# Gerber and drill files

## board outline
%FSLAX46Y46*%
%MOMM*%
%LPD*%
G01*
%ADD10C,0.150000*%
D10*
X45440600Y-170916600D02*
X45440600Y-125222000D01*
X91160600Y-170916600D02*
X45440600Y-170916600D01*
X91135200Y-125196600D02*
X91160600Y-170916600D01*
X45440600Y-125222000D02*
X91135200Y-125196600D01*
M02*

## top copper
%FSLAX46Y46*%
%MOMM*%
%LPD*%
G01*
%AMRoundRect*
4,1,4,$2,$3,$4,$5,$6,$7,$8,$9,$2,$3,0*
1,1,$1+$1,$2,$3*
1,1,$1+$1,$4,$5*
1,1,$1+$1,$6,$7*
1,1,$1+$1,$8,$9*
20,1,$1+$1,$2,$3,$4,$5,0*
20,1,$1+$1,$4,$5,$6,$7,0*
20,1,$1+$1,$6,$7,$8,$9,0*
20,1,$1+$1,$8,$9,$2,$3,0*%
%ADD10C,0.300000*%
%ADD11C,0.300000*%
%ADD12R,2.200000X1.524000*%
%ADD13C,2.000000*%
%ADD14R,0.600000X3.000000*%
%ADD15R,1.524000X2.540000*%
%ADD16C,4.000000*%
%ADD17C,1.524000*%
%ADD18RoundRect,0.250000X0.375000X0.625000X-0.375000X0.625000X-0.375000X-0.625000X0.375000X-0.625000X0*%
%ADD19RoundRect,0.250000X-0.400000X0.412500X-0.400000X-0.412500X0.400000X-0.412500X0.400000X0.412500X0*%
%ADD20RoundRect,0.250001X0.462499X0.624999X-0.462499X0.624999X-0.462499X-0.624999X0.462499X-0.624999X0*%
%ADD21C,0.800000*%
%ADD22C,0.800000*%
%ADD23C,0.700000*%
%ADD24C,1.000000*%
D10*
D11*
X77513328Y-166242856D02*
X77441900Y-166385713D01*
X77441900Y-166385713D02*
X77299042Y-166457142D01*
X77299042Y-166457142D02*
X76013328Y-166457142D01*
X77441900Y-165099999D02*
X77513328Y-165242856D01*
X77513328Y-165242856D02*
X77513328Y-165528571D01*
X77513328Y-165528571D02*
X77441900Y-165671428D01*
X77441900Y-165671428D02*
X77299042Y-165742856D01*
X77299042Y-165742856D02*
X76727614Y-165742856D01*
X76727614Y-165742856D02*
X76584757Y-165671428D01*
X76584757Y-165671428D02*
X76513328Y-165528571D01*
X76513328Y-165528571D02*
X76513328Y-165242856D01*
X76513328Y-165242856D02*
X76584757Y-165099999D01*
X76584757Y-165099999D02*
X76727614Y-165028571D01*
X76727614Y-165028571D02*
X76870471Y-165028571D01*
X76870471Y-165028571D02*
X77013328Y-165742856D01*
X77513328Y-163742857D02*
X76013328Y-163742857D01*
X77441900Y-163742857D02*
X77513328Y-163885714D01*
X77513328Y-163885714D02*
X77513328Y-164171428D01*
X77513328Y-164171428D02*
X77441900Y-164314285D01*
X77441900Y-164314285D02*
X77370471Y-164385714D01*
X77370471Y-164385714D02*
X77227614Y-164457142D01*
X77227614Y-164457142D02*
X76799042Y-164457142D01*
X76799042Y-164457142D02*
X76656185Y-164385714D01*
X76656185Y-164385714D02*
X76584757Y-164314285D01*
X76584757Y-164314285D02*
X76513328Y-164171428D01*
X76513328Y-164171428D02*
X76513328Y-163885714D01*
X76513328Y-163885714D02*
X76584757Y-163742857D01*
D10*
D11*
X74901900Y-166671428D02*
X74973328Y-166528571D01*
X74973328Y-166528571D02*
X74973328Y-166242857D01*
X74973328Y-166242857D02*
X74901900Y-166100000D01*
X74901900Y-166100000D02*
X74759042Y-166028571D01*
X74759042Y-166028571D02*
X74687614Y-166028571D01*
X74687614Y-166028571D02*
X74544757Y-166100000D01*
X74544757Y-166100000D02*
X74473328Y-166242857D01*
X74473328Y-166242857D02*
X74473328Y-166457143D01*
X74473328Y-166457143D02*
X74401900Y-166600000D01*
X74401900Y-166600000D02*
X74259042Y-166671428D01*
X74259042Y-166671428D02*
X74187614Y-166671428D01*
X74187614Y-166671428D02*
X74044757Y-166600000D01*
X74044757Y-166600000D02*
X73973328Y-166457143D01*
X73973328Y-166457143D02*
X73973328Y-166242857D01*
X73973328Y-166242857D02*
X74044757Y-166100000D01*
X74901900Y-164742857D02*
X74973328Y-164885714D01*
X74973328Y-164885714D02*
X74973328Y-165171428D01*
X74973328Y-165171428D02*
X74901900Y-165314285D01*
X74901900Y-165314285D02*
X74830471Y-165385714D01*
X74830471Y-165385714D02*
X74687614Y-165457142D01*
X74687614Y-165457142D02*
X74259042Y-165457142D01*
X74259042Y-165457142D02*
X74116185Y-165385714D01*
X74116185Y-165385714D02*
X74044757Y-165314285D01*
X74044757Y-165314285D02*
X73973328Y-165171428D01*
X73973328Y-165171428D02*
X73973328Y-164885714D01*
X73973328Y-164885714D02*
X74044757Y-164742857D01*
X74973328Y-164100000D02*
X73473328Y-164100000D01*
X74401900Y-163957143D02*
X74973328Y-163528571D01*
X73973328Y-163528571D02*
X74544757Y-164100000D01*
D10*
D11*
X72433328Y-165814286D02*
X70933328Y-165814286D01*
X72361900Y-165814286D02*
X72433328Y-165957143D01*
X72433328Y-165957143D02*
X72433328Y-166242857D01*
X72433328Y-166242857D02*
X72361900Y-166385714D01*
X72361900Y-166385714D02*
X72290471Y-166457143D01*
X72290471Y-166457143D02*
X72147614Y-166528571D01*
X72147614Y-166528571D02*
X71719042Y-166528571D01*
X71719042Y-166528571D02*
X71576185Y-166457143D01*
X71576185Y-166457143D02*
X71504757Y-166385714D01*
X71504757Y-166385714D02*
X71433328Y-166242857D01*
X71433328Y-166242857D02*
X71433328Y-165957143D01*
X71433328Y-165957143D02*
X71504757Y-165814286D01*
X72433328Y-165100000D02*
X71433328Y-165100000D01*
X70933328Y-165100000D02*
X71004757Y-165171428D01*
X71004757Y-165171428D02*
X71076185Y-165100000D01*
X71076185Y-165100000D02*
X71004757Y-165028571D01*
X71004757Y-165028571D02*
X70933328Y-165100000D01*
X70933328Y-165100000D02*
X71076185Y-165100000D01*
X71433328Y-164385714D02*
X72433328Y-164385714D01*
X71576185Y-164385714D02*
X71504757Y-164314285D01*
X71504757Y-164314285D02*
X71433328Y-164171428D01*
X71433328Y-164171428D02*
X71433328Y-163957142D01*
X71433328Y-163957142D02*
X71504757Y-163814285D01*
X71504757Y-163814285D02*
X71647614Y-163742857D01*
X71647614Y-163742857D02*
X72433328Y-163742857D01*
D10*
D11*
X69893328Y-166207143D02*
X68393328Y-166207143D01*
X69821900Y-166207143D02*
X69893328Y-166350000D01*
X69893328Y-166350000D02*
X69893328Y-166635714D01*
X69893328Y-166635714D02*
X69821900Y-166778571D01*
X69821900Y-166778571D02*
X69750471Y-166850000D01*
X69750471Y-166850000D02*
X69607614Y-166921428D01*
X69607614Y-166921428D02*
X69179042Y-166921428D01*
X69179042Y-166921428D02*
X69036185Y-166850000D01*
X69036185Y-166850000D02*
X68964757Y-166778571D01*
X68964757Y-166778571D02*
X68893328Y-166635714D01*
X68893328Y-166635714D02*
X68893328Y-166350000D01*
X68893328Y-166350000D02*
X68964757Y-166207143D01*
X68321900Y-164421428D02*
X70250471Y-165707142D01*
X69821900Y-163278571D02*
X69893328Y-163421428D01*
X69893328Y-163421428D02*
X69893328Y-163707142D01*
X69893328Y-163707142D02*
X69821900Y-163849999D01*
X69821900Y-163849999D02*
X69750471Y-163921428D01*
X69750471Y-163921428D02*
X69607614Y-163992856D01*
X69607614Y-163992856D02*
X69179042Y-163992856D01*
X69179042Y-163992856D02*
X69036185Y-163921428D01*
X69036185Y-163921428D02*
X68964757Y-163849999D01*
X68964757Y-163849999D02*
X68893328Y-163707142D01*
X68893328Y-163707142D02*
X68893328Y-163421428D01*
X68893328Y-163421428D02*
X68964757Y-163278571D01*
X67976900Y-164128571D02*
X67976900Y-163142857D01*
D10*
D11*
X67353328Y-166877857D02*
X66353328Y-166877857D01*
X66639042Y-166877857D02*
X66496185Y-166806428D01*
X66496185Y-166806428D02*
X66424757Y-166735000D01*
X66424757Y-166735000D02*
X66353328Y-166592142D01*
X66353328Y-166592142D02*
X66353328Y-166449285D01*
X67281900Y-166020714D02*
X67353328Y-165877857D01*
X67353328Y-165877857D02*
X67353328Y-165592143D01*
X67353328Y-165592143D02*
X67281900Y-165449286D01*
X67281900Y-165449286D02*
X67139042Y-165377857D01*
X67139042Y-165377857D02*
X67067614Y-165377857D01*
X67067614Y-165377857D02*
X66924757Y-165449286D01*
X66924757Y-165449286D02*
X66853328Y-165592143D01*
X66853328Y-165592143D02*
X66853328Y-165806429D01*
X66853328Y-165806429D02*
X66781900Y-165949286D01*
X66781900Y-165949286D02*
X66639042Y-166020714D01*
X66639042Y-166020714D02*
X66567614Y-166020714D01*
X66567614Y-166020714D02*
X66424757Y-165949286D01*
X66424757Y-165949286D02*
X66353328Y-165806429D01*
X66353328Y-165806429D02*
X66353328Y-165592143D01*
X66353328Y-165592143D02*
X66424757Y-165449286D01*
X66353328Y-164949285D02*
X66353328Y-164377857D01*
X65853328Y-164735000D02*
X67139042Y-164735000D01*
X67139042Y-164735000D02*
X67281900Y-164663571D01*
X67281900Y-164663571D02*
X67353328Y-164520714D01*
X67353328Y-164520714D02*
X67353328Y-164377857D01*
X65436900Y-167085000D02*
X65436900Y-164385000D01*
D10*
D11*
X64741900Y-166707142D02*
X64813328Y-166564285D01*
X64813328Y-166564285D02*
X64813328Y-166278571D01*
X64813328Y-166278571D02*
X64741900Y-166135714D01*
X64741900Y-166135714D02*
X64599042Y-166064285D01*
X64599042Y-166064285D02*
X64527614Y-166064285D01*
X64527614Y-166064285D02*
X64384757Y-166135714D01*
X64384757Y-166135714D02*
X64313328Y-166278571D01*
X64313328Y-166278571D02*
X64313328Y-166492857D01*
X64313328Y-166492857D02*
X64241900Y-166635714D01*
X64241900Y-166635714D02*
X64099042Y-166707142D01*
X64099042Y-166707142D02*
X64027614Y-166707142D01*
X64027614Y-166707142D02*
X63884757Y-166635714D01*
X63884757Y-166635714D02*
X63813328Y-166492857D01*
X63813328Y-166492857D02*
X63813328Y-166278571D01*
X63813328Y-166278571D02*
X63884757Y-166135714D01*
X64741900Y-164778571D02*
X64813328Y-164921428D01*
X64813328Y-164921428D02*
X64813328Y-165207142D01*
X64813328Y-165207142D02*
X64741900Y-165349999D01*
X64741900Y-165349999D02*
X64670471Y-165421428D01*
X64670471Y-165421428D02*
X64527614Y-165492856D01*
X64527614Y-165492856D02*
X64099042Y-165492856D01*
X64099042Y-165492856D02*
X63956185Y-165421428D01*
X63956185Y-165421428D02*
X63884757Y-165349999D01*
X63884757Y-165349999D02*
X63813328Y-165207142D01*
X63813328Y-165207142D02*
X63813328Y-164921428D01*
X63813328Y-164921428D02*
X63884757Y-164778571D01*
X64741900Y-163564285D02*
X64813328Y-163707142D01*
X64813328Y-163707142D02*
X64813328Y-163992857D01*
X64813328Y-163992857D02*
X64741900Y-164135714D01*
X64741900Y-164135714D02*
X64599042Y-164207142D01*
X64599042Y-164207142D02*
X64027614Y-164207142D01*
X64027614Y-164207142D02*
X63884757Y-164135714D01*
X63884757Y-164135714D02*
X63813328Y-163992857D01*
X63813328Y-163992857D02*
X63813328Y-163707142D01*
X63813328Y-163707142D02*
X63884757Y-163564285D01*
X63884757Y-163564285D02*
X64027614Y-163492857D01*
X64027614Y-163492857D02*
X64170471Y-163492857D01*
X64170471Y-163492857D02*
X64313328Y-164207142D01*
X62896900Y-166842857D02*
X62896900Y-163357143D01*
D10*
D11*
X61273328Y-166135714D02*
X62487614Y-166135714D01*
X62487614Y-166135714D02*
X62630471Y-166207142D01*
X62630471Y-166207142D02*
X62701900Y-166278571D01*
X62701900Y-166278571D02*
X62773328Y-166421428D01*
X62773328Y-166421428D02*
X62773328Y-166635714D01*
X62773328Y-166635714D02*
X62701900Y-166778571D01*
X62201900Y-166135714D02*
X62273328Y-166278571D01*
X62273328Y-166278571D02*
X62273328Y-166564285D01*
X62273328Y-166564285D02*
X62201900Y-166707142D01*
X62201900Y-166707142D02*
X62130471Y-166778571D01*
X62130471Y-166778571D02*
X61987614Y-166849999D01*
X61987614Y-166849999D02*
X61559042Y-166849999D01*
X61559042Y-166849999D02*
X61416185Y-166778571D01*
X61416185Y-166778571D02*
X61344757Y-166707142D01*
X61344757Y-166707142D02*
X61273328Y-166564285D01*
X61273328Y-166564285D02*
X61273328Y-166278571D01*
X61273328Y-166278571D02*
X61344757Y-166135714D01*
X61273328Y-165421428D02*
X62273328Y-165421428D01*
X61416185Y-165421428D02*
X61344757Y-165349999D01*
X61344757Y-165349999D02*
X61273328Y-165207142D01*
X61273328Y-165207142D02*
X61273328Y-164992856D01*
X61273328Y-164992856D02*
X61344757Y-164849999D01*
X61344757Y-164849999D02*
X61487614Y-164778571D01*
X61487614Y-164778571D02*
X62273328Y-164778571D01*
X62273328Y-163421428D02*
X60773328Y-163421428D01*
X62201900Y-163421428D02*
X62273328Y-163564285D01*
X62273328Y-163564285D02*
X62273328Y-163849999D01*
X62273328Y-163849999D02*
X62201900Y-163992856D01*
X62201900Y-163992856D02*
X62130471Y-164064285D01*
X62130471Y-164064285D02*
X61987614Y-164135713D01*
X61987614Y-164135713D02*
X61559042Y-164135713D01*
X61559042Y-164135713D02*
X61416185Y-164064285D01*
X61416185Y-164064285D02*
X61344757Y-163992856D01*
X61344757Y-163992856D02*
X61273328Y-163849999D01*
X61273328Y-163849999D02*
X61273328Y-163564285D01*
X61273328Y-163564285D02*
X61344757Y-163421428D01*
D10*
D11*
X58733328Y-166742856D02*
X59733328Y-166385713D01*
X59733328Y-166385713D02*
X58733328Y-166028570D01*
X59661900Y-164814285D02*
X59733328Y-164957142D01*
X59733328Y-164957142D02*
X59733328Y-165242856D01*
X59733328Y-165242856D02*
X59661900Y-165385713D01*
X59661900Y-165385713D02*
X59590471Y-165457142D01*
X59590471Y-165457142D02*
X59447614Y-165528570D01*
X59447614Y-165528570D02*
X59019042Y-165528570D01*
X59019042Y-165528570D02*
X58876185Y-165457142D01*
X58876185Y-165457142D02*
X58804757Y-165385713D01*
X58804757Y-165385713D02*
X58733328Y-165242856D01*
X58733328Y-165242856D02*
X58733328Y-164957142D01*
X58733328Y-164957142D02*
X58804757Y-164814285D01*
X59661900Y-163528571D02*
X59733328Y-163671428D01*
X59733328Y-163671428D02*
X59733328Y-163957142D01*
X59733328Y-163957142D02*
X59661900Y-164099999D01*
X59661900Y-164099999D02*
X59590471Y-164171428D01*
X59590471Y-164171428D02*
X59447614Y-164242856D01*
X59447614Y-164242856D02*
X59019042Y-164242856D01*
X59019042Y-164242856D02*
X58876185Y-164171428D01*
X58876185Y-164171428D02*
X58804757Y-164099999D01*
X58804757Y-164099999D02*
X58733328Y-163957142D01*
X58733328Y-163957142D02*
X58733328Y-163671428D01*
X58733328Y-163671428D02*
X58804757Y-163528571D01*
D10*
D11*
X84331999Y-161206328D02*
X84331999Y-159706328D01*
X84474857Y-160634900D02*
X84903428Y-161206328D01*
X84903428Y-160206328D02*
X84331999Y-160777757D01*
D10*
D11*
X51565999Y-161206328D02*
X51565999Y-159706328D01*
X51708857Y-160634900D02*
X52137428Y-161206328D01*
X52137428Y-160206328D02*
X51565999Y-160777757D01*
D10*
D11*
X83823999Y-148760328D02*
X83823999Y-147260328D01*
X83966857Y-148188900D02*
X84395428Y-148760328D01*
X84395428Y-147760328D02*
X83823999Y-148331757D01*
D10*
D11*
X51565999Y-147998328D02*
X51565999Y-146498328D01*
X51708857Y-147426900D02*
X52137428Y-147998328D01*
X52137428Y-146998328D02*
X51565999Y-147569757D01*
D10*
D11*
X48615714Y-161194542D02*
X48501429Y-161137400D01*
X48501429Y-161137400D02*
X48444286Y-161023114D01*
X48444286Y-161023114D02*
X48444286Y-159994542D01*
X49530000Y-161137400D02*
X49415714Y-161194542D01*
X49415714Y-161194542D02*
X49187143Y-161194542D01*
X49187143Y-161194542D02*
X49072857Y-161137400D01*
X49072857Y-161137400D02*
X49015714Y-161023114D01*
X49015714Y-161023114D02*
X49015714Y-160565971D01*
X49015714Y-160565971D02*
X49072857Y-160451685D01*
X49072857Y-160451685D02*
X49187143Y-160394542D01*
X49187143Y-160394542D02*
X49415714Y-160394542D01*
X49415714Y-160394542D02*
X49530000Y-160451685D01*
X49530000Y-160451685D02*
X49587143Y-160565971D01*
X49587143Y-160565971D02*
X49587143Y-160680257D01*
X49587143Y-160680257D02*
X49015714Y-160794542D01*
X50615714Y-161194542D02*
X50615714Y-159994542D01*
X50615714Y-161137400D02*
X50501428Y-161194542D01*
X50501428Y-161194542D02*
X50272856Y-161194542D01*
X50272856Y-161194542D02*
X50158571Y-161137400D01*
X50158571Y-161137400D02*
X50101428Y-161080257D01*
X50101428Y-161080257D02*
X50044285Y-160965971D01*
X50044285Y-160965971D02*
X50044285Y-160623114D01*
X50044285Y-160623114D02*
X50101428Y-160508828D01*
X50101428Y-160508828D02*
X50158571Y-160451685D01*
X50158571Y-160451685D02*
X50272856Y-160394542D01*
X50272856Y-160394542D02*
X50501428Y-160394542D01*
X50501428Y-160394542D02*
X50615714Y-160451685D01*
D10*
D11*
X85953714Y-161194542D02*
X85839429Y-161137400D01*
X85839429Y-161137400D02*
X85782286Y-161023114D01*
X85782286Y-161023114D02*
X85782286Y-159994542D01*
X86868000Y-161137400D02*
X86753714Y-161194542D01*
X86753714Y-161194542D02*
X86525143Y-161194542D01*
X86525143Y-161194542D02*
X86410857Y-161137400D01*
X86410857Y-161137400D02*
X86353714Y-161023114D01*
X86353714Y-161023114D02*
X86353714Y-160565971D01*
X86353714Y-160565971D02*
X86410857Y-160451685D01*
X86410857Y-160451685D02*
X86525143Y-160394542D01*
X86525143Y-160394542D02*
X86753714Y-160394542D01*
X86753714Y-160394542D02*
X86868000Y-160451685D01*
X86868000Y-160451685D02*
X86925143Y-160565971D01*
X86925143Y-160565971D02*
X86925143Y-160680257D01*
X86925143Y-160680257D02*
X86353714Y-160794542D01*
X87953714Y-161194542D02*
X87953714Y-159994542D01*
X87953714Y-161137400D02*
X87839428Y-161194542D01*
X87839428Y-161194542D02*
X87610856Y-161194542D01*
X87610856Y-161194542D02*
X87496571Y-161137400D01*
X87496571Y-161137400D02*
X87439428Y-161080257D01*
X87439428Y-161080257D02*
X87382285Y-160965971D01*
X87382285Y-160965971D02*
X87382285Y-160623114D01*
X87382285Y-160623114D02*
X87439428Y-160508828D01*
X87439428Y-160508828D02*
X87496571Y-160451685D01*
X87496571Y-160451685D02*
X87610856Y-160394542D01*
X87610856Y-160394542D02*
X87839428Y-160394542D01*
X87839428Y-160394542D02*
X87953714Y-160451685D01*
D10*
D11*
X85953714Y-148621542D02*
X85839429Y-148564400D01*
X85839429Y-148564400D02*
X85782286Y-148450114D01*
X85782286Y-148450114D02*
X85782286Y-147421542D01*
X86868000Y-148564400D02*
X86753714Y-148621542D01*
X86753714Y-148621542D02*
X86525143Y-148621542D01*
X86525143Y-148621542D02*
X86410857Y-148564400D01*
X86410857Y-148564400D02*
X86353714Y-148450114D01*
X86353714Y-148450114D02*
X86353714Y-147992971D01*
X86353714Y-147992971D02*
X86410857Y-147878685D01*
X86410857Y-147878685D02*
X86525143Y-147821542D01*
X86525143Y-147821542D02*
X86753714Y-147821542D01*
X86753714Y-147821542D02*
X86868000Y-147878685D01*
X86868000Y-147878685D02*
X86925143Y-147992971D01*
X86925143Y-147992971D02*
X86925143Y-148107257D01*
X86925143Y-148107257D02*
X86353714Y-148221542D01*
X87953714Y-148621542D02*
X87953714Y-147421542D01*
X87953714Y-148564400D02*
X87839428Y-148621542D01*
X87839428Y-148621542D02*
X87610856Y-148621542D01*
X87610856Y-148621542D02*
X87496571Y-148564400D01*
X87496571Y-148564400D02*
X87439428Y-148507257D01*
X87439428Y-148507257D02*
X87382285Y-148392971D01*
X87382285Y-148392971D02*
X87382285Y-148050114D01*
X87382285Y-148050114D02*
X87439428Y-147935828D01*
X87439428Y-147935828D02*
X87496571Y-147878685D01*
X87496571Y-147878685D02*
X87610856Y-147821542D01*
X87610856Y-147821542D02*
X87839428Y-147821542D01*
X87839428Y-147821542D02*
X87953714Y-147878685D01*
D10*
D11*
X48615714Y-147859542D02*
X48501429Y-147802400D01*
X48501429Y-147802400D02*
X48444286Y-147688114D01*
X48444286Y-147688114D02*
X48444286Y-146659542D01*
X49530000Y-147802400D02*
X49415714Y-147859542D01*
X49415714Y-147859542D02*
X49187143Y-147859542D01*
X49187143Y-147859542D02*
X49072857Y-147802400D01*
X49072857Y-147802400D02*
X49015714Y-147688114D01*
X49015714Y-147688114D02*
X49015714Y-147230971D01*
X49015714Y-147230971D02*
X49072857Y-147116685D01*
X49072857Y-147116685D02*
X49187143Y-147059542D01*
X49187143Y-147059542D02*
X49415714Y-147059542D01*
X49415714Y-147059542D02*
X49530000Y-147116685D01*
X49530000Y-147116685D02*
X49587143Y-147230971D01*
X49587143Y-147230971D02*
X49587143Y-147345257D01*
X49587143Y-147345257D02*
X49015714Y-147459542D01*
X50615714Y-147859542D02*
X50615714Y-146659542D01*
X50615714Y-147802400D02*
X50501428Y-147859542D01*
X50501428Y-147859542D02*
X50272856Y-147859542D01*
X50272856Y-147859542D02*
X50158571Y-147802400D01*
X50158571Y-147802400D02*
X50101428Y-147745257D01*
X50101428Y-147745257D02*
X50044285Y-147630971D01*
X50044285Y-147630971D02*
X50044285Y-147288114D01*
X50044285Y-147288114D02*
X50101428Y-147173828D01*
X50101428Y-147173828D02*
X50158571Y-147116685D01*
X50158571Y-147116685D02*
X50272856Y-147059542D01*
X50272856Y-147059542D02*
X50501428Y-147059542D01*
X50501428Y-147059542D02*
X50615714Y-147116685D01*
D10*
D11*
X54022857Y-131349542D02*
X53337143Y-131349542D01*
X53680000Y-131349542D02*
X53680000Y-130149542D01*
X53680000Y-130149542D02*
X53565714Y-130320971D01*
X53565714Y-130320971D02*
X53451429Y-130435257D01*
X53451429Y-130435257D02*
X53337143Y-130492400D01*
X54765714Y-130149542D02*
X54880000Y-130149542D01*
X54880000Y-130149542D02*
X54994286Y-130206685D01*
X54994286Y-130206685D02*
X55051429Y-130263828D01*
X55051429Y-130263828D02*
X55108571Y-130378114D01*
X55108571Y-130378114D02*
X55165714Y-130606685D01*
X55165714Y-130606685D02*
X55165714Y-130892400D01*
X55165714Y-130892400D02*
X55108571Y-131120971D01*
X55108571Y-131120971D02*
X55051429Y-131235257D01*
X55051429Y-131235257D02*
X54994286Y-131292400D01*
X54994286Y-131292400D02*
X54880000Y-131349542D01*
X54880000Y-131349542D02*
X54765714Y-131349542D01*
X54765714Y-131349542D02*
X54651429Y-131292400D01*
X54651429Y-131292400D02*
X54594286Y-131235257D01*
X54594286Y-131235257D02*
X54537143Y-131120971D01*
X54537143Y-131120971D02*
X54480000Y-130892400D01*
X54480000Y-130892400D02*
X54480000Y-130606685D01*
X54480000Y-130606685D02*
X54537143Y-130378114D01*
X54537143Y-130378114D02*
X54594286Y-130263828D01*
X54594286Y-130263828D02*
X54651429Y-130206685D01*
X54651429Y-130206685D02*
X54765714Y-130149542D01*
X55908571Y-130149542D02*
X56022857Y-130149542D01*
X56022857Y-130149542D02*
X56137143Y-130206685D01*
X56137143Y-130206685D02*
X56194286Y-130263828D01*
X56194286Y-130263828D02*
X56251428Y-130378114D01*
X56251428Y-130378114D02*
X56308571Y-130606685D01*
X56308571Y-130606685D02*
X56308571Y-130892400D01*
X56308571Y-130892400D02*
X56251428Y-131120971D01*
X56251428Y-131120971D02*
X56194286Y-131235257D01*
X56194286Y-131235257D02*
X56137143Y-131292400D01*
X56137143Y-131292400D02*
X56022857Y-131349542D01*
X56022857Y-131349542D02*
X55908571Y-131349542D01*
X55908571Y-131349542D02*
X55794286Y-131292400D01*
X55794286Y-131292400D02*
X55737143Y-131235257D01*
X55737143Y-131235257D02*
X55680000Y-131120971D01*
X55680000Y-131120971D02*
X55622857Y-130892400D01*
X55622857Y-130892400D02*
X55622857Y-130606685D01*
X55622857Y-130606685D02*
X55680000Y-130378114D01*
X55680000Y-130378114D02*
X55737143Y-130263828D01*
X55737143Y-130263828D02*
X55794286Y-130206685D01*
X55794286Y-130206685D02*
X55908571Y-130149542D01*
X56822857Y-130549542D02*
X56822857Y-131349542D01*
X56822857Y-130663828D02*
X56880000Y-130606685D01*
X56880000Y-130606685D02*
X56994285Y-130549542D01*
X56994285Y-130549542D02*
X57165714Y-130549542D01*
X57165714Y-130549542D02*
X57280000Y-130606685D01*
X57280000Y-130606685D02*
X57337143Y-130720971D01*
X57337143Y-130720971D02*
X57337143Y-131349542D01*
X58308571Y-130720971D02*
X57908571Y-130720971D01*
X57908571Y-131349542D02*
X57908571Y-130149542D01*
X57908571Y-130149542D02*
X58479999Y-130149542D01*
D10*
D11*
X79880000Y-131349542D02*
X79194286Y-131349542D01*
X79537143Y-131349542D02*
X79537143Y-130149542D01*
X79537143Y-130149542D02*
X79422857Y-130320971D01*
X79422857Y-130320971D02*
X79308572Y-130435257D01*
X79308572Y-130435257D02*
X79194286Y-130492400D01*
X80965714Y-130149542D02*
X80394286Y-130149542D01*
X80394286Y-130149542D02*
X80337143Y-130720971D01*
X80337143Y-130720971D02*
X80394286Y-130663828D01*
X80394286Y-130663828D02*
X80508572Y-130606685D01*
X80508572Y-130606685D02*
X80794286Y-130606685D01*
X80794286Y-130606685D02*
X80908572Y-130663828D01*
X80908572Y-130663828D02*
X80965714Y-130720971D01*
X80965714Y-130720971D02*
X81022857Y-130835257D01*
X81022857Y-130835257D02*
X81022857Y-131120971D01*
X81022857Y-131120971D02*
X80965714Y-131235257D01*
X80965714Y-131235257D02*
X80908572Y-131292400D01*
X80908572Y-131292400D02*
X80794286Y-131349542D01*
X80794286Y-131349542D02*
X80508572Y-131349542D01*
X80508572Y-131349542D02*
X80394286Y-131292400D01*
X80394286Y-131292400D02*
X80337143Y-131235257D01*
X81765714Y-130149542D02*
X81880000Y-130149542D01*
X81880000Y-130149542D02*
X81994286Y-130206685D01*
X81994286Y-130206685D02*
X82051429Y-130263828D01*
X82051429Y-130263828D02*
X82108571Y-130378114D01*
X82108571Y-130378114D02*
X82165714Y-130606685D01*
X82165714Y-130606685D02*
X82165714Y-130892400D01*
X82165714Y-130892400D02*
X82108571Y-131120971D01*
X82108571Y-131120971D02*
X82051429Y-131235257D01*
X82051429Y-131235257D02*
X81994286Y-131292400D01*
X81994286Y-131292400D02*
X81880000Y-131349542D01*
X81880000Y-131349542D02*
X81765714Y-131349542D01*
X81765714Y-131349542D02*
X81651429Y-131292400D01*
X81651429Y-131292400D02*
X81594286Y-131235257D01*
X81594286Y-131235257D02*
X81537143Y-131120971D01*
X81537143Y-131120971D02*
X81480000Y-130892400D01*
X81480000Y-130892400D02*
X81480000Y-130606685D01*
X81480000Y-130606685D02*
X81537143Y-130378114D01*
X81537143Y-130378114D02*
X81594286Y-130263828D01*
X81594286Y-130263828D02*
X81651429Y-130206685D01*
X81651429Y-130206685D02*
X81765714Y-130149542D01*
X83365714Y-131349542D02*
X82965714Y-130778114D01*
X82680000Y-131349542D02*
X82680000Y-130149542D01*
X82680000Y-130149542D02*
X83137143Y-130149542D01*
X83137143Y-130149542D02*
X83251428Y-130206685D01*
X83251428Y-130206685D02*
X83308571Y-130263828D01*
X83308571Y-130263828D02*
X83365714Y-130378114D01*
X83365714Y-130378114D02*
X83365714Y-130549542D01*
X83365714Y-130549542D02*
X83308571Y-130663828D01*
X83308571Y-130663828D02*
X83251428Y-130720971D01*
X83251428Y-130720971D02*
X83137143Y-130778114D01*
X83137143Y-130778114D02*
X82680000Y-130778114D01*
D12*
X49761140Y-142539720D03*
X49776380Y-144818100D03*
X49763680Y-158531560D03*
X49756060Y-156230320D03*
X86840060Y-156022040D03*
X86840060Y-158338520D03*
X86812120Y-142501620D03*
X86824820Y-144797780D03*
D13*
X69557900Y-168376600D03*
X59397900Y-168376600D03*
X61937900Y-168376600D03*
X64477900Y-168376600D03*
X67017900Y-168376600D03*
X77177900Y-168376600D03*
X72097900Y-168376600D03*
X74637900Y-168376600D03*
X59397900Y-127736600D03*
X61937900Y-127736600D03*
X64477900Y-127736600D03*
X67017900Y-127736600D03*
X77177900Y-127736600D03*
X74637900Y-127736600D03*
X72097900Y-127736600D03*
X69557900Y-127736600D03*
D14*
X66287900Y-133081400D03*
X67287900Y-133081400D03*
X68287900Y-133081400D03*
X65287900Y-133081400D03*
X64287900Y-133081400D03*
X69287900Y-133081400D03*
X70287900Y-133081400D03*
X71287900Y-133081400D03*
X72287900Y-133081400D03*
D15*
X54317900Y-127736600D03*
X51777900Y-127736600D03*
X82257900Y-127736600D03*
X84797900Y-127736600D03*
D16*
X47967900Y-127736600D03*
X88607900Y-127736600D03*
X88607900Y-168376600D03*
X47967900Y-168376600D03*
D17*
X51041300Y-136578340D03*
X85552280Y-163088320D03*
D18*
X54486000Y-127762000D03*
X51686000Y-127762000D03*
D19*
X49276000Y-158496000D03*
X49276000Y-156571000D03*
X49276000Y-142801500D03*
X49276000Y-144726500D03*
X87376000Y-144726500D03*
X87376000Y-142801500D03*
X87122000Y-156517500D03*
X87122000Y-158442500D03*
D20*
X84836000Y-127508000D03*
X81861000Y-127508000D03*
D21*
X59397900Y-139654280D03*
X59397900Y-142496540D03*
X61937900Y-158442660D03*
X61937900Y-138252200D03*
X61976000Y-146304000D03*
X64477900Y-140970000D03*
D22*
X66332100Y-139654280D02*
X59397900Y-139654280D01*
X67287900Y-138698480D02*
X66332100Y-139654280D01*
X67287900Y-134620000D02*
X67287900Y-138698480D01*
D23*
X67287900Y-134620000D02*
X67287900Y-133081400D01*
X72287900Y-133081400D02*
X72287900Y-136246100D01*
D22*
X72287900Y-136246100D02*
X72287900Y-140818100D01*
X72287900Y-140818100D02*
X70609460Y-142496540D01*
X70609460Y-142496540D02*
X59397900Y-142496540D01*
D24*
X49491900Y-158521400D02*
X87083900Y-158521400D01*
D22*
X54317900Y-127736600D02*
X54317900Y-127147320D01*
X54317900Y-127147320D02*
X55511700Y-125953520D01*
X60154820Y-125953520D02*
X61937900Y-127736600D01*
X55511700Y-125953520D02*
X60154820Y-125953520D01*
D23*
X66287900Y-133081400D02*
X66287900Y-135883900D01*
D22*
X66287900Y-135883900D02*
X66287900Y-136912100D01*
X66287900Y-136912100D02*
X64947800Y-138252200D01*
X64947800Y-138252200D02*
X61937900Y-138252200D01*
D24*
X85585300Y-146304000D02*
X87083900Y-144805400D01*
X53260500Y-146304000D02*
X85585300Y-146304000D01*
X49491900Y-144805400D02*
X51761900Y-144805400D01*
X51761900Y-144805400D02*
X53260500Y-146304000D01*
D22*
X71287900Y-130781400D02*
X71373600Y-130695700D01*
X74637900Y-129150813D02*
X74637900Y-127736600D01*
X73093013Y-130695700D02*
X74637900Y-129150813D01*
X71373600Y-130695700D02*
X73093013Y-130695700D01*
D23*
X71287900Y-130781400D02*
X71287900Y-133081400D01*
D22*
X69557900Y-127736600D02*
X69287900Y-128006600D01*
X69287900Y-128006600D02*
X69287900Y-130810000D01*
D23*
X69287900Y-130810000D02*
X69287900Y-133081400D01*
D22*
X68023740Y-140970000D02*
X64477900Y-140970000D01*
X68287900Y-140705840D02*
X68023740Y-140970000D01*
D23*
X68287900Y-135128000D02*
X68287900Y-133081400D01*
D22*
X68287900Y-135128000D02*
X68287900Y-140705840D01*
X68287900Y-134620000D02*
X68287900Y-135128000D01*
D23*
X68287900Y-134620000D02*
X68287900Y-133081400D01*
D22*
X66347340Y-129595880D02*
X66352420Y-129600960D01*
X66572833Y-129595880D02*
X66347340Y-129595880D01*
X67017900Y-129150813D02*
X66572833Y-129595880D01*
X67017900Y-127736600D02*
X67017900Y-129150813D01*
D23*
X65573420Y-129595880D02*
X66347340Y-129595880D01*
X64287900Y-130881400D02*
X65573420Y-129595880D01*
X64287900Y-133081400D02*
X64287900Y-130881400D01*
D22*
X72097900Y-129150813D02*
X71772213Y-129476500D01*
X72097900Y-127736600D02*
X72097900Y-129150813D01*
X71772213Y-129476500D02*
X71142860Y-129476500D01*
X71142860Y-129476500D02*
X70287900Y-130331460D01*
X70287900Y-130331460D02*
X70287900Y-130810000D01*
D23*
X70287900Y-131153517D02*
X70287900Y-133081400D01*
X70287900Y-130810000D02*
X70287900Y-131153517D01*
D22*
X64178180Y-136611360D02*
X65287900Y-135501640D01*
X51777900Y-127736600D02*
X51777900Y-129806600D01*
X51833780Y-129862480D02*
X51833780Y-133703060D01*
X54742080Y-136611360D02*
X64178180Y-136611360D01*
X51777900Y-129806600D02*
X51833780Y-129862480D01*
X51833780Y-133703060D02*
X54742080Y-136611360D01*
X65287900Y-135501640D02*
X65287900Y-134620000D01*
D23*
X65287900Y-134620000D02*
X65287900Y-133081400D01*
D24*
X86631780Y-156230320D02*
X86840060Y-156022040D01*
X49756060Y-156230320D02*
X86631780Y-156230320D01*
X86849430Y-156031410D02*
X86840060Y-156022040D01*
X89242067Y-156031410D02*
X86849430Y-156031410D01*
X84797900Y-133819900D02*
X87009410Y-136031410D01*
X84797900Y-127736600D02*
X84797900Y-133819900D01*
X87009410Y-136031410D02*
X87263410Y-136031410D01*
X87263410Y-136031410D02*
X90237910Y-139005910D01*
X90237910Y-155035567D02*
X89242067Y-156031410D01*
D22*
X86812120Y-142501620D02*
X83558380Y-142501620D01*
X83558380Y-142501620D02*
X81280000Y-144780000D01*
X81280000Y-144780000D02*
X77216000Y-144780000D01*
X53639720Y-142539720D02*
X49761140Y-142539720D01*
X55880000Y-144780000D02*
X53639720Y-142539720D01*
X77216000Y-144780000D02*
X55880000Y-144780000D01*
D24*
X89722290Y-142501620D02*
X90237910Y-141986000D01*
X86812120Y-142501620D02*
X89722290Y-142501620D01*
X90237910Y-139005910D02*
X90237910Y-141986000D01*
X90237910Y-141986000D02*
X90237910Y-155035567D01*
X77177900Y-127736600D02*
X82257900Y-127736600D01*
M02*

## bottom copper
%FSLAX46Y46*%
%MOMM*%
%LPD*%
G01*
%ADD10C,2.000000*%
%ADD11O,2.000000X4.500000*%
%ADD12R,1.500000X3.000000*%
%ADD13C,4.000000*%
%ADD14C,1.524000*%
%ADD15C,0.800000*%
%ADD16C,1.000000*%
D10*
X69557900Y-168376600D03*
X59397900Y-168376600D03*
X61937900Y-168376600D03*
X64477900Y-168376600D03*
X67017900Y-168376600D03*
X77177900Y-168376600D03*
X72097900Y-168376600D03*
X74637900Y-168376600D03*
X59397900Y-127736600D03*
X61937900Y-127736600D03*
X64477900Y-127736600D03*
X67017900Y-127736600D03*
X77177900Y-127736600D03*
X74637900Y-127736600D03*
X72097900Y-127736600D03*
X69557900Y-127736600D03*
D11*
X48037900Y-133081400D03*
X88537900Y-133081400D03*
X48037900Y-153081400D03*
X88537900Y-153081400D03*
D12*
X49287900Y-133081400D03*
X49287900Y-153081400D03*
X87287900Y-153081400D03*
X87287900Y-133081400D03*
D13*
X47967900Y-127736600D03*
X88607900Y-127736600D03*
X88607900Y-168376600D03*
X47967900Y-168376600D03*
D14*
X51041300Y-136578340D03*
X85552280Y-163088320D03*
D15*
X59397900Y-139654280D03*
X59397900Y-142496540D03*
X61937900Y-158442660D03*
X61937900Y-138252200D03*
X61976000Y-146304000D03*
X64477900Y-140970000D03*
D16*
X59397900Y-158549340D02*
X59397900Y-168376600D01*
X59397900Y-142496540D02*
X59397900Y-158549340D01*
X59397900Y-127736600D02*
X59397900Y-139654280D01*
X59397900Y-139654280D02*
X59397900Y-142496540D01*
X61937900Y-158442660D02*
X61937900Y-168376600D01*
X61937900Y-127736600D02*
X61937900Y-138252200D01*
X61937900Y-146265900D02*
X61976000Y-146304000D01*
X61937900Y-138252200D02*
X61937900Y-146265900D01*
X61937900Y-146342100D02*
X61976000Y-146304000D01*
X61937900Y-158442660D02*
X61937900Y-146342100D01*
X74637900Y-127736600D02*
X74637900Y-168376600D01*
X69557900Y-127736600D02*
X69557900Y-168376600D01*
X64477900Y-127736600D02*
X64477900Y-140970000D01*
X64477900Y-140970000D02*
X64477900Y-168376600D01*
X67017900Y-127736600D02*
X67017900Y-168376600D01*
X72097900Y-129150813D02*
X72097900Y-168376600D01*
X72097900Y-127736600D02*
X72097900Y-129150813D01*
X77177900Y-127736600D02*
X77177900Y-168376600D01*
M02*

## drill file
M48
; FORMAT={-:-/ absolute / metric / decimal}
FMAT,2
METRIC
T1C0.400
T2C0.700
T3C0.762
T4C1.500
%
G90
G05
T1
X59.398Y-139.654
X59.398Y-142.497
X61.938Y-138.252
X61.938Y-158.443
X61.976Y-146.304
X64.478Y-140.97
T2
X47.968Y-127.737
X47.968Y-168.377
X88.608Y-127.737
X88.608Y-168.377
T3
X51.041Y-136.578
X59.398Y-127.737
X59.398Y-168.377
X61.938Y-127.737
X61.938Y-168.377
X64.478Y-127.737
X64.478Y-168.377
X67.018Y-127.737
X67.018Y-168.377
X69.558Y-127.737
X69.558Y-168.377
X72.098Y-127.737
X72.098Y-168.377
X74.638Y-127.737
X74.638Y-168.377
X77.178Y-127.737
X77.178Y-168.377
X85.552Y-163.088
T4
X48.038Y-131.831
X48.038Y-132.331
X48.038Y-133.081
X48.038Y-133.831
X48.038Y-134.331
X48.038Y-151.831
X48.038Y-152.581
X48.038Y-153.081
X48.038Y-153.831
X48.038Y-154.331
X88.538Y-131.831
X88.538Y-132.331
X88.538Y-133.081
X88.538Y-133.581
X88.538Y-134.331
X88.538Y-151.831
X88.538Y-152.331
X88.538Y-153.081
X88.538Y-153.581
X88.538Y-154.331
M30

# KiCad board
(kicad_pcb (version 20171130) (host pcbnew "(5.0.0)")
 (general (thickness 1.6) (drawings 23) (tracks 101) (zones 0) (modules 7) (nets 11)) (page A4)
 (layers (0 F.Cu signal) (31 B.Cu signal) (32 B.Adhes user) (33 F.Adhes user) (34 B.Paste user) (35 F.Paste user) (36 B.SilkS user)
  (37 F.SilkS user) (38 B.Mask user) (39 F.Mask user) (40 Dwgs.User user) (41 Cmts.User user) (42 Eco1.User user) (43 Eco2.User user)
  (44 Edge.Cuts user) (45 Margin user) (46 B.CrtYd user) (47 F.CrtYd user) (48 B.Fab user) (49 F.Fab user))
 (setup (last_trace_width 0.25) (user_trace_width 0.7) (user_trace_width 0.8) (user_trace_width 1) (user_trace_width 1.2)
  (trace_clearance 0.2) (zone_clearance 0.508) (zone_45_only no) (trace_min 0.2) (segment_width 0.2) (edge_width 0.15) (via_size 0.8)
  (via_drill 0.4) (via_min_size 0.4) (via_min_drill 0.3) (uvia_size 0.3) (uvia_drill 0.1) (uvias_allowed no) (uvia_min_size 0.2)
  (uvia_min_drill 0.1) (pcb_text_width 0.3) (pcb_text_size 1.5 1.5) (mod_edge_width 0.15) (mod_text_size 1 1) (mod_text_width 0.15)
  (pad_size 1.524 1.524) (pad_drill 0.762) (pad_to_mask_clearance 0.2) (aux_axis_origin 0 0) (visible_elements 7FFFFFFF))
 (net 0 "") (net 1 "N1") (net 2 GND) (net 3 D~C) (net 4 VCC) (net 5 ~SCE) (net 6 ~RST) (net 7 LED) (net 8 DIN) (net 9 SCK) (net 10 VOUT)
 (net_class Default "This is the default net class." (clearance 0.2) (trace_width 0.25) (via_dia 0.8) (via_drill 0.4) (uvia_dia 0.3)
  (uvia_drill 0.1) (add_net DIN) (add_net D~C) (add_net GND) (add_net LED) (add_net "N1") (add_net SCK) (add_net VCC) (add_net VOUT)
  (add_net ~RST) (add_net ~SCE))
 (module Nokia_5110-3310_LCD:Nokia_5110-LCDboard (layer F.Cu) (at 68.2879 146.7866)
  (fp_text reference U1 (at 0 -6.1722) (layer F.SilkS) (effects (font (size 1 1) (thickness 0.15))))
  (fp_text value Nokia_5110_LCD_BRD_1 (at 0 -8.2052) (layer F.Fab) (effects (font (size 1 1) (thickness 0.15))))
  (pad 15 smd rect (at -18.52676 -4.24688 180) (size 2.2 1.524) (layers F.Cu F.Paste F.Mask) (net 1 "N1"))
  (pad 16 smd rect (at -18.51152 -1.9685) (size 2.2 1.524) (layers F.Cu F.Paste F.Mask) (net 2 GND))
  (pad 18 smd rect (at -18.52422 11.74496) (size 2.2 1.524) (layers F.Cu F.Paste F.Mask) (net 2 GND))
  (pad 17 smd rect (at -18.53184 9.44372) (size 2.2 1.524) (layers F.Cu F.Paste F.Mask) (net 1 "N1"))
  (pad 21 smd rect (at 18.55216 9.23544) (size 2.2 1.524) (layers F.Cu F.Paste F.Mask) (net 1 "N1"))
  (pad 22 smd rect (at 18.55216 11.55192) (size 2.2 1.524) (layers F.Cu F.Paste F.Mask) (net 2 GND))
  (pad 19 smd rect (at 18.52422 -4.28498) (size 2.2 1.524) (layers F.Cu F.Paste F.Mask) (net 1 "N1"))
  (pad 20 smd rect (at 18.53692 -1.98882) (size 2.2 1.524) (layers F.Cu F.Paste F.Mask) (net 2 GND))
  (pad 45 thru_hole circle (at 1.27 21.59) (size 2 2) (drill 0.762) (layers *.Cu *.Mask) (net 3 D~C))
  (pad 41 thru_hole circle (at -8.89 21.59) (size 2 2) (drill 0.762) (layers *.Cu *.Mask) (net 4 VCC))
  (pad 42 thru_hole circle (at -6.35 21.59) (size 2 2) (drill 0.762) (layers *.Cu *.Mask) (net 2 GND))
  (pad 43 thru_hole circle (at -3.81 21.59) (size 2 2) (drill 0.762) (layers *.Cu *.Mask) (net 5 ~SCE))
  (pad 44 thru_hole circle (at -1.27 21.59) (size 2 2) (drill 0.762) (layers *.Cu *.Mask) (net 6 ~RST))
  (pad 48 thru_hole circle (at 8.89 21.59) (size 2 2) (drill 0.762) (layers *.Cu *.Mask) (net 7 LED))
  (pad 46 thru_hole circle (at 3.81 21.59) (size 2 2) (drill 0.762) (layers *.Cu *.Mask) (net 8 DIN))
  (pad 47 thru_hole circle (at 6.35 21.59) (size 2 2) (drill 0.762) (layers *.Cu *.Mask) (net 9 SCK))
  (pad 31 thru_hole circle (at -8.89 -19.05) (size 2 2) (drill 0.762) (layers *.Cu *.Mask) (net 4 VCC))
  (pad 32 thru_hole circle (at -6.35 -19.05) (size 2 2) (drill 0.762) (layers *.Cu *.Mask) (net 2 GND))
  (pad 33 thru_hole circle (at -3.81 -19.05) (size 2 2) (drill 0.762) (layers *.Cu *.Mask) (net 5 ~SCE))
  (pad 34 thru_hole circle (at -1.27 -19.05) (size 2 2) (drill 0.762) (layers *.Cu *.Mask) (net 6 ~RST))
  (pad 38 thru_hole circle (at 8.89 -19.05) (size 2 2) (drill 0.762) (layers *.Cu *.Mask) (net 7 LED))
  (pad 37 thru_hole circle (at 6.35 -19.05) (size 2 2) (drill 0.762) (layers *.Cu *.Mask) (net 9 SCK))
  (pad 36 thru_hole circle (at 3.81 -19.05) (size 2 2) (drill 0.762) (layers *.Cu *.Mask) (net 8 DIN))
  (pad 35 thru_hole circle (at 1.27 -19.05) (size 2 2) (drill 0.762) (layers *.Cu *.Mask) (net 3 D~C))
  (pad "" np_thru_hole circle (at 20.25 -14.4552) (size 1.5 1.5) (drill 1.5) (layers *.Mask B.Cu F.SilkS))
  (pad "" np_thru_hole circle (at 20.25 -12.4552) (size 1.5 1.5) (drill 1.5) (layers *.Mask B.Cu F.SilkS))
  (pad "" np_thru_hole circle (at 20.25 -14.9552) (size 1.5 1.5) (drill 1.5) (layers *.Mask B.Cu F.SilkS))
  (pad 3 smd rect (at -2 -13.7052) (size 0.6 3) (layers F.Cu F.Paste F.Mask) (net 2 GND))
  (pad 4 smd rect (at -1 -13.7052) (size 0.6 3) (layers F.Cu F.Paste F.Mask) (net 4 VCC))
  (pad 5 smd rect (at 0 -13.7052) (size 0.6 3) (layers F.Cu F.Paste F.Mask) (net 5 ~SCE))
  (pad 2 smd rect (at -3 -13.7052) (size 0.6 3) (layers F.Cu F.Paste F.Mask) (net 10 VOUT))
  (pad 1 smd rect (at -4 -13.7052) (size 0.6 3) (layers F.Cu F.Paste F.Mask) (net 6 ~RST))
  (pad 6 smd rect (at 1 -13.7052) (size 0.6 3) (layers F.Cu F.Paste F.Mask) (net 3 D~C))
  (pad 7 smd rect (at 2 -13.7052) (size 0.6 3) (layers F.Cu F.Paste F.Mask) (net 8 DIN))
  (pad 8 smd rect (at 3 -13.7052) (size 0.6 3) (layers F.Cu F.Paste F.Mask) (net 9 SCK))
  (pad 9 smd rect (at 4 -13.7052) (size 0.6 3) (layers F.Cu F.Paste F.Mask) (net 4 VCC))
  (pad "" np_thru_hole oval (at -20.25 -13.7052) (size 2 4.5) (drill 1.5) (layers *.Mask B.Cu F.SilkS))
  (pad "" np_thru_hole oval (at 20.25 -13.7052) (size 2 4.5) (drill 1.5) (layers *.Mask B.Cu F.SilkS))
  (pad "" np_thru_hole oval (at -20.25 6.2948) (size 2 4.5) (drill 1.5) (layers *.Mask B.Cu F.SilkS))
  (pad "" np_thru_hole oval (at 20.25 6.2948) (size 2 4.5) (drill 1.5) (layers *.Mask B.Cu F.SilkS))
  (pad "" smd rect (at -19 -13.7052) (size 1.5 3) (layers B.Cu B.Paste B.Mask))
  (pad "" smd rect (at -19 6.2948) (size 1.5 3) (layers B.Cu B.Paste B.Mask))
  (pad "" smd rect (at 19 6.2948) (size 1.5 3) (layers B.Cu B.Paste B.Mask))
  (pad "" smd rect (at 19 -13.7052) (size 1.5 3) (layers B.Cu B.Paste B.Mask))
  (pad "" np_thru_hole circle (at 20.25 -13.2052) (size 1.5 1.5) (drill 1.5) (layers *.Mask B.Cu F.SilkS))
  (pad "" np_thru_hole circle (at 20.25 5.0448) (size 1.5 1.5) (drill 1.5) (layers *.Mask B.Cu F.SilkS))
  (pad "" np_thru_hole circle (at 20.25 7.5448) (size 1.5 1.5) (drill 1.5) (layers *.Mask B.Cu F.SilkS))
  (pad "" np_thru_hole circle (at -20.25 -14.4552) (size 1.5 1.5) (drill 1.5) (layers *.Mask B.Cu F.SilkS))
  (pad "" np_thru_hole circle (at -20.25 -14.9552) (size 1.5 1.5) (drill 1.5) (layers *.Mask B.Cu F.SilkS))
  (pad "" np_thru_hole circle (at -20.25 -12.9552) (size 1.5 1.5) (drill 1.5) (layers *.Mask B.Cu F.SilkS))
  (pad "" np_thru_hole circle (at -20.25 -12.4552) (size 1.5 1.5) (drill 1.5) (layers *.Mask B.Cu F.SilkS))
  (pad "" np_thru_hole circle (at -20.25 5.0448) (size 1.5 1.5) (drill 1.5) (layers *.Mask B.Cu F.SilkS))
  (pad "" np_thru_hole circle (at -20.25 7.5448) (size 1.5 1.5) (drill 1.5) (layers *.Mask B.Cu F.SilkS))
  (pad "" np_thru_hole circle (at -20.25 5.7948) (size 1.5 1.5) (drill 1.5) (layers *.Mask B.Cu F.SilkS))
  (pad "" np_thru_hole circle (at -20.25 7.0448) (size 1.5 1.5) (drill 1.5) (layers *.Mask B.Cu F.SilkS))
  (pad "" np_thru_hole circle (at 20.25 5.5448) (size 1.5 1.5) (drill 1.5) (layers *.Mask B.Cu F.SilkS))
  (pad "" np_thru_hole circle (at 20.25 6.7948) (size 1.5 1.5) (drill 1.5) (layers *.Mask B.Cu F.SilkS))
  (pad 12 smd rect (at -13.97 -19.05 90) (size 2.54 1.524) (layers F.Cu F.Paste F.Mask) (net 2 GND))
  (pad 11 smd rect (at -16.51 -19.05 90) (size 2.54 1.524) (layers F.Cu F.Paste F.Mask) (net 10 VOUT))
  (pad 13 smd rect (at 13.97 -19.05 90) (size 2.54 1.524) (layers F.Cu F.Paste F.Mask) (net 7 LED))
  (pad 14 smd rect (at 16.51 -19.05 90) (size 2.54 1.524) (layers F.Cu F.Paste F.Mask) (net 1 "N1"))
  (pad 01 thru_hole circle (at -20.32 -19.05 90) (size 4 4) (drill 0.7) (layers *.Cu *.Adhes *.Paste *.Mask))
  (pad 02 thru_hole circle (at 20.32 -19.05 90) (size 4 4) (drill 0.7) (layers *.Cu *.Adhes *.Paste *.Mask))
  (pad 04 thru_hole circle (at 20.32 21.59 90) (size 4 4) (drill 0.7) (layers *.Cu *.Adhes *.Paste *.Mask))
  (pad 03 thru_hole circle (at -20.32 21.59 90) (size 4 4) (drill 0.7) (layers *.Cu *.Adhes *.Paste *.Mask))
  (pad 10 thru_hole circle (at -17.2466 -10.20826) (size 1.524 1.524) (drill 0.762) (layers *.Cu *.Mask))
  (pad 23 thru_hole circle (at 17.26438 16.30172) (size 1.524 1.524) (drill 0.762) (layers *.Cu *.Mask)))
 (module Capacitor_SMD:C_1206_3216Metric (layer F.Cu) (at 53.086 127.762 180)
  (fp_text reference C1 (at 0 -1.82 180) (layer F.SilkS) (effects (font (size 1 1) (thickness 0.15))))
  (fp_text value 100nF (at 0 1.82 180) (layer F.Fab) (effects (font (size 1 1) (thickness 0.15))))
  (pad 1 smd roundrect (at -1.4 0 180) (size 1.25 1.75) (layers F.Cu F.Paste F.Mask) (roundrect_rratio 0.2) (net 2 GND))
  (pad 2 smd roundrect (at 1.4 0 180) (size 1.25 1.75) (layers F.Cu F.Paste F.Mask) (roundrect_rratio 0.2) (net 10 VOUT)))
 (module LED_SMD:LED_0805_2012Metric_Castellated (layer F.Cu) (at 49.276 157.5335 270)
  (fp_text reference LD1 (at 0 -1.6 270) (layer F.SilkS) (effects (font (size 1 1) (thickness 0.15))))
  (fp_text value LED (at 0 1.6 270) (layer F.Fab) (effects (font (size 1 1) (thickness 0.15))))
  (pad 2 smd roundrect (at 0.9625 0 270) (size 1.325 1.3) (layers F.Cu F.Paste F.Mask) (roundrect_rratio 0.192308) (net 2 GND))
  (pad 1 smd roundrect (at -0.9625 0 270) (size 1.325 1.3) (layers F.Cu F.Paste F.Mask) (roundrect_rratio 0.192308) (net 1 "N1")))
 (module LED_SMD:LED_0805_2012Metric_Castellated (layer F.Cu) (at 49.276 143.764 270)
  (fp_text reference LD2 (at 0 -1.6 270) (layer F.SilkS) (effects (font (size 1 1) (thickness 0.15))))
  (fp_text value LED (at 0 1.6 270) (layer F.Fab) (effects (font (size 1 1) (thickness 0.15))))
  (pad 1 smd roundrect (at -0.9625 0 270) (size 1.325 1.3) (layers F.Cu F.Paste F.Mask) (roundrect_rratio 0.192308) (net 1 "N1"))
  (pad 2 smd roundrect (at 0.9625 0 270) (size 1.325 1.3) (layers F.Cu F.Paste F.Mask) (roundrect_rratio 0.192308) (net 2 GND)))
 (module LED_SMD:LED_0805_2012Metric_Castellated (layer F.Cu) (at 87.376 143.764 270)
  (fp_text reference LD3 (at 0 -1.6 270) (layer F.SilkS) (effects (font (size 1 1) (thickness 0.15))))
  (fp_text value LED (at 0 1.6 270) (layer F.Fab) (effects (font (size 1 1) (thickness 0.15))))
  (pad 2 smd roundrect (at 0.9625 0 270) (size 1.325 1.3) (layers F.Cu F.Paste F.Mask) (roundrect_rratio 0.192308) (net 2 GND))
  (pad 1 smd roundrect (at -0.9625 0 270) (size 1.325 1.3) (layers F.Cu F.Paste F.Mask) (roundrect_rratio 0.192308) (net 1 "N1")))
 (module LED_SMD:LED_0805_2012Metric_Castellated (layer F.Cu) (at 87.122 157.48 270)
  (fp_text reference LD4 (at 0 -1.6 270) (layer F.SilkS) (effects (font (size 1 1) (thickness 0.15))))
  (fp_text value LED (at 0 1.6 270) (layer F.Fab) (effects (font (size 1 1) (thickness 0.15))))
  (pad 1 smd roundrect (at -0.9625 0 270) (size 1.325 1.3) (layers F.Cu F.Paste F.Mask) (roundrect_rratio 0.192308) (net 1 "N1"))
  (pad 2 smd roundrect (at 0.9625 0 270) (size 1.325 1.3) (layers F.Cu F.Paste F.Mask) (roundrect_rratio 0.192308) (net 2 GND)))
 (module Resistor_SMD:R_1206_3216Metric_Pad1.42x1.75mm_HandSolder (layer F.Cu) (at 83.3485 127.508 180)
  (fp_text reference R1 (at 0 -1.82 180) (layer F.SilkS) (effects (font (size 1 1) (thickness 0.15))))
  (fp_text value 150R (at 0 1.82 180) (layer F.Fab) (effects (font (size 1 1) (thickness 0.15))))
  (pad 1 smd roundrect (at -1.4875 0 180) (size 1.425 1.75) (layers F.Cu F.Paste F.Mask) (roundrect_rratio 0.175439) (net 1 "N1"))
  (pad 2 smd roundrect (at 1.4875 0 180) (size 1.425 1.75) (layers F.Cu F.Paste F.Mask) (roundrect_rratio 0.175439) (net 7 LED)))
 (gr_line (start 45.4406 170.9166) (end 45.4406 125.222) (layer Edge.Cuts) (width 0.15))
 (gr_line (start 91.1606 170.9166) (end 45.4406 170.9166) (layer Edge.Cuts) (width 0.15))
 (gr_line (start 91.1352 125.1966) (end 91.1606 170.9166) (layer Edge.Cuts) (width 0.15))
 (gr_line (start 45.4406 125.222) (end 91.1352 125.1966) (layer Edge.Cuts) (width 0.15))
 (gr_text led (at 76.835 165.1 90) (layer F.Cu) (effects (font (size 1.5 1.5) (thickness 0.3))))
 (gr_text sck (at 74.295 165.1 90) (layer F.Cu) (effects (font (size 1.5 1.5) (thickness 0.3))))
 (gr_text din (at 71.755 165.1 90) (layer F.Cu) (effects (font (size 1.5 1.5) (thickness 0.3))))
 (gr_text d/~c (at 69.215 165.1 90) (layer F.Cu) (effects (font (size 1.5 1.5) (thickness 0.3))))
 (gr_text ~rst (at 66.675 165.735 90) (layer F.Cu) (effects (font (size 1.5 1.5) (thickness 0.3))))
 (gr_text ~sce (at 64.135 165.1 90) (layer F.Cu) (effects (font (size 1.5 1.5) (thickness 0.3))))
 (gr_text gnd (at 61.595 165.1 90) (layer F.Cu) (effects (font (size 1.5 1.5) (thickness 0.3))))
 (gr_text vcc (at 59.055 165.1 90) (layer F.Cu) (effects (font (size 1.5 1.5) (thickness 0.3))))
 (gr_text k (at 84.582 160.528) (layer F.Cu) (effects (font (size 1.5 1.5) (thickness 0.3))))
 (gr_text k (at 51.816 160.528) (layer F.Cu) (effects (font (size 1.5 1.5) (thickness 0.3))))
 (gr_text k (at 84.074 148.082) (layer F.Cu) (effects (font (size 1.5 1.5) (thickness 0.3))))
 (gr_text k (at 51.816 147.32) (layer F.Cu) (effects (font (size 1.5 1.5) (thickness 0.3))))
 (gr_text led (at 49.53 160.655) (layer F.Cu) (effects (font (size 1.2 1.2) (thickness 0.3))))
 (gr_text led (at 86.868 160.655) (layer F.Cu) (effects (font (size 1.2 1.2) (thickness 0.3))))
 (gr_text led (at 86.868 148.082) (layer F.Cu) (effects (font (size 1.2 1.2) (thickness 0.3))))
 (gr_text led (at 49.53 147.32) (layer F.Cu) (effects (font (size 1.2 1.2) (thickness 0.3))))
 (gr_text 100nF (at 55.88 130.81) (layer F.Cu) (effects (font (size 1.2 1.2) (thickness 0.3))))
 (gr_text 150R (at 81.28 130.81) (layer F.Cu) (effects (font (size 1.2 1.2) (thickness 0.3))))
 (segment (start 59.3979 158.54934) (end 59.3979 168.3766) (width 1) (layer B.Cu) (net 4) (status 20))
 (segment (start 59.3979 142.49654) (end 59.3979 158.54934) (width 1) (layer B.Cu) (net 4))
 (via (at 59.3979 139.65428) (size 0.8) (drill 0.4) (layers F.Cu B.Cu) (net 4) (status 1000000))
 (segment (start 66.3321 139.65428) (end 59.3979 139.65428) (width 0.8) (layer F.Cu) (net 4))
 (segment (start 67.2879 138.69848) (end 66.3321 139.65428) (width 0.8) (layer F.Cu) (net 4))
 (segment (start 59.3979 127.7366) (end 59.3979 139.65428) (width 1) (layer B.Cu) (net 4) (status 10))
 (segment (start 59.3979 139.65428) (end 59.3979 142.49654) (width 1) (layer B.Cu) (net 4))
 (segment (start 67.2879 134.62) (end 67.2879 138.69848) (width 0.8) (layer F.Cu) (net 4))
 (segment (start 67.2879 134.62) (end 67.2879 133.0814) (width 0.7) (layer F.Cu) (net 4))
 (segment (start 72.2879 133.0814) (end 72.2879 136.2461) (width 0.7) (layer F.Cu) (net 4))
 (segment (start 72.2879 136.2461) (end 72.2879 140.8181) (width 0.8) (layer F.Cu) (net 4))
 (via (at 59.3979 142.49654) (size 0.8) (drill 0.4) (layers F.Cu B.Cu) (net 4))
 (segment (start 72.2879 140.8181) (end 70.60946 142.49654) (width 0.8) (layer F.Cu) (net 4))
 (segment (start 70.60946 142.49654) (end 59.3979 142.49654) (width 0.8) (layer F.Cu) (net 4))
 (segment (start 49.4919 158.5214) (end 87.0839 158.5214) (width 1) (layer F.Cu) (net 2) (status 30))
 (segment (start 61.9379 158.44266) (end 61.9379 168.3766) (width 1) (layer B.Cu) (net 2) (status 20))
 (via (at 61.9379 158.44266) (size 0.8) (drill 0.4) (layers F.Cu B.Cu) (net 2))
 (segment (start 54.3179 127.7366) (end 54.3179 127.14732) (width 0.8) (layer F.Cu) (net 2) (status 30))
 (segment (start 54.3179 127.14732) (end 55.5117 125.95352) (width 0.8) (layer F.Cu) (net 2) (status 10))
 (segment (start 60.15482 125.95352) (end 61.9379 127.7366) (width 0.8) (layer F.Cu) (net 2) (status 20))
 (segment (start 55.5117 125.95352) (end 60.15482 125.95352) (width 0.8) (layer F.Cu) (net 2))
 (segment (start 61.9379 127.7366) (end 61.9379 138.2522) (width 1) (layer B.Cu) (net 2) (status 10))
 (segment (start 66.2879 133.0814) (end 66.2879 135.8839) (width 0.7) (layer F.Cu) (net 2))
 (segment (start 66.2879 135.8839) (end 66.2879 136.9121) (width 0.8) (layer F.Cu) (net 2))
 (via (at 61.9379 138.2522) (size 0.8) (drill 0.4) (layers F.Cu B.Cu) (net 2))
 (segment (start 66.2879 136.9121) (end 64.9478 138.2522) (width 0.8) (layer F.Cu) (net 2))
 (segment (start 64.9478 138.2522) (end 61.9379 138.2522) (width 0.8) (layer F.Cu) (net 2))
 (segment (start 85.5853 146.304) (end 87.0839 144.8054) (width 1) (layer F.Cu) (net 2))
 (segment (start 53.2605 146.304) (end 85.5853 146.304) (width 1) (layer F.Cu) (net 2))
 (segment (start 49.4919 144.8054) (end 51.7619 144.8054) (width 1) (layer F.Cu) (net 2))
 (segment (start 51.7619 144.8054) (end 53.2605 146.304) (width 1) (layer F.Cu) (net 2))
 (via (at 61.976 146.304) (size 0.8) (drill 0.4) (layers F.Cu B.Cu) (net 2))
 (segment (start 61.9379 146.2659) (end 61.976 146.304) (width 1) (layer B.Cu) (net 2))
 (segment (start 61.9379 138.2522) (end 61.9379 146.2659) (width 1) (layer B.Cu) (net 2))
 (segment (start 61.9379 146.3421) (end 61.976 146.304) (width 1) (layer B.Cu) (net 2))
 (segment (start 61.9379 158.44266) (end 61.9379 146.3421) (width 1) (layer B.Cu) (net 2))
 (segment (start 74.6379 127.7366) (end 74.6379 168.3766) (width 1) (layer B.Cu) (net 9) (status 30))
 (segment (start 71.2879 130.7814) (end 71.3736 130.6957) (width 0.8) (layer F.Cu) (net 9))
 (segment (start 74.6379 129.150813) (end 74.6379 127.7366) (width 0.8) (layer F.Cu) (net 9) (status 20))
 (segment (start 73.093013 130.6957) (end 74.6379 129.150813) (width 0.8) (layer F.Cu) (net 9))
 (segment (start 71.3736 130.6957) (end 73.093013 130.6957) (width 0.8) (layer F.Cu) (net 9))
 (segment (start 71.2879 130.7814) (end 71.2879 133.0814) (width 0.7) (layer F.Cu) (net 9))
 (segment (start 69.5579 127.7366) (end 69.5579 168.3766) (width 1) (layer B.Cu) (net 3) (status 30))
 (segment (start 69.5579 127.7366) (end 69.2879 128.0066) (width 0.8) (layer F.Cu) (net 3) (status 30))
 (segment (start 69.2879 128.0066) (end 69.2879 130.81) (width 0.8) (layer F.Cu) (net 3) (status 10))
 (segment (start 69.2879 130.81) (end 69.2879 133.0814) (width 0.7) (layer F.Cu) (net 3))
 (via (at 64.4779 140.97) (size 0.8) (drill 0.4) (layers F.Cu B.Cu) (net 5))
 (segment (start 68.02374 140.97) (end 64.4779 140.97) (width 0.8) (layer F.Cu) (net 5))
 (segment (start 68.2879 140.70584) (end 68.02374 140.97) (width 0.8) (layer F.Cu) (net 5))
 (segment (start 64.4779 127.7366) (end 64.4779 140.97) (width 1) (layer B.Cu) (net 5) (status 10))
 (segment (start 64.4779 140.97) (end 64.4779 168.3766) (width 1) (layer B.Cu) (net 5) (status 20))
 (segment (start 68.2879 135.128) (end 68.2879 133.0814) (width 0.7) (layer F.Cu) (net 5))
 (segment (start 68.2879 135.128) (end 68.2879 140.70584) (width 0.8) (layer F.Cu) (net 5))
 (segment (start 68.2879 134.62) (end 68.2879 135.128) (width 0.8) (layer F.Cu) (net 5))
 (segment (start 68.2879 134.62) (end 68.2879 133.0814) (width 0.7) (layer F.Cu) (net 5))
 (segment (start 67.0179 127.7366) (end 67.0179 168.3766) (width 1) (layer B.Cu) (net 6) (status 30))
 (segment (start 66.34734 129.59588) (end 66.35242 129.60096) (width 0.8) (layer F.Cu) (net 6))
 (segment (start 66.572833 129.59588) (end 66.34734 129.59588) (width 0.8) (layer F.Cu) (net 6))
 (segment (start 67.0179 129.150813) (end 66.572833 129.59588) (width 0.8) (layer F.Cu) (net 6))
 (segment (start 67.0179 127.7366) (end 67.0179 129.150813) (width 0.8) (layer F.Cu) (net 6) (status 10))
 (segment (start 65.57342 129.59588) (end 66.34734 129.59588) (width 0.7) (layer F.Cu) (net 6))
 (segment (start 64.2879 130.8814) (end 65.57342 129.59588) (width 0.7) (layer F.Cu) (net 6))
 (segment (start 64.2879 133.0814) (end 64.2879 130.8814) (width 0.7) (layer F.Cu) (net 6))
 (segment (start 72.0979 129.150813) (end 72.0979 168.3766) (width 1) (layer B.Cu) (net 8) (status 20))
 (segment (start 72.0979 127.7366) (end 72.0979 129.150813) (width 1) (layer B.Cu) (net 8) (status 10))
 (segment (start 72.0979 129.150813) (end 71.772213 129.4765) (width 0.8) (layer F.Cu) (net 8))
 (segment (start 72.0979 127.7366) (end 72.0979 129.150813) (width 0.8) (layer F.Cu) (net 8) (status 10))
 (segment (start 71.772213 129.4765) (end 71.14286 129.4765) (width 0.8) (layer F.Cu) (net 8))
 (segment (start 71.14286 129.4765) (end 70.2879 130.33146) (width 0.8) (layer F.Cu) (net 8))
 (segment (start 70.2879 130.33146) (end 70.2879 130.81) (width 0.8) (layer F.Cu) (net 8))
 (segment (start 70.2879 131.153517) (end 70.2879 133.0814) (width 0.7) (layer F.Cu) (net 8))
 (segment (start 70.2879 130.81) (end 70.2879 131.153517) (width 0.7) (layer F.Cu) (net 8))
 (segment (start 64.17818 136.61136) (end 65.2879 135.50164) (width 0.8) (layer F.Cu) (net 10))
 (segment (start 51.7779 127.7366) (end 51.7779 129.8066) (width 0.8) (layer F.Cu) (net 10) (status 10))
 (segment (start 51.83378 129.86248) (end 51.83378 133.70306) (width 0.8) (layer F.Cu) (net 10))
 (segment (start 54.74208 136.61136) (end 64.17818 136.61136) (width 0.8) (layer F.Cu) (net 10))
 (segment (start 51.7779 129.8066) (end 51.83378 129.86248) (width 0.8) (layer F.Cu) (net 10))
 (segment (start 51.83378 133.70306) (end 54.74208 136.61136) (width 0.8) (layer F.Cu) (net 10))
 (segment (start 65.2879 135.50164) (end 65.2879 134.62) (width 0.8) (layer F.Cu) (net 10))
 (segment (start 65.2879 134.62) (end 65.2879 133.0814) (width 0.7) (layer F.Cu) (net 10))
 (segment (start 86.63178 156.23032) (end 86.84006 156.02204) (width 1) (layer F.Cu) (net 1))
 (segment (start 49.75606 156.23032) (end 86.63178 156.23032) (width 1) (layer F.Cu) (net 1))
 (segment (start 86.84943 156.03141) (end 86.84006 156.02204) (width 1) (layer F.Cu) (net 1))
 (segment (start 89.242067 156.03141) (end 86.84943 156.03141) (width 1) (layer F.Cu) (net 1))
 (segment (start 84.7979 133.8199) (end 87.00941 136.03141) (width 1) (layer F.Cu) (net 1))
 (segment (start 84.7979 127.7366) (end 84.7979 133.8199) (width 1) (layer F.Cu) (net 1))
 (segment (start 87.00941 136.03141) (end 87.26341 136.03141) (width 1) (layer F.Cu) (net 1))
 (segment (start 87.26341 136.03141) (end 90.23791 139.00591) (width 1) (layer F.Cu) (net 1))
 (segment (start 90.23791 155.035567) (end 89.242067 156.03141) (width 1) (layer F.Cu) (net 1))
 (segment (start 86.81212 142.50162) (end 83.55838 142.50162) (width 0.8) (layer F.Cu) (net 1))
 (segment (start 83.55838 142.50162) (end 81.28 144.78) (width 0.8) (layer F.Cu) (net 1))
 (segment (start 81.28 144.78) (end 77.216 144.78) (width 0.8) (layer F.Cu) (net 1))
 (segment (start 53.63972 142.53972) (end 49.76114 142.53972) (width 0.8) (layer F.Cu) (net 1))
 (segment (start 55.88 144.78) (end 53.63972 142.53972) (width 0.8) (layer F.Cu) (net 1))
 (segment (start 77.216 144.78) (end 55.88 144.78) (width 0.8) (layer F.Cu) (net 1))
 (segment (start 89.72229 142.50162) (end 90.23791 141.986) (width 1) (layer F.Cu) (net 1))
 (segment (start 86.81212 142.50162) (end 89.72229 142.50162) (width 1) (layer F.Cu) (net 1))
 (segment (start 90.23791 139.00591) (end 90.23791 141.986) (width 1) (layer F.Cu) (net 1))
 (segment (start 90.23791 141.986) (end 90.23791 155.035567) (width 1) (layer F.Cu) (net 1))
 (segment (start 77.1779 127.7366) (end 82.2579 127.7366) (width 1) (layer F.Cu) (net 7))
 (segment (start 77.1779 127.7366) (end 77.1779 168.3766) (width 1) (layer B.Cu) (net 7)))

